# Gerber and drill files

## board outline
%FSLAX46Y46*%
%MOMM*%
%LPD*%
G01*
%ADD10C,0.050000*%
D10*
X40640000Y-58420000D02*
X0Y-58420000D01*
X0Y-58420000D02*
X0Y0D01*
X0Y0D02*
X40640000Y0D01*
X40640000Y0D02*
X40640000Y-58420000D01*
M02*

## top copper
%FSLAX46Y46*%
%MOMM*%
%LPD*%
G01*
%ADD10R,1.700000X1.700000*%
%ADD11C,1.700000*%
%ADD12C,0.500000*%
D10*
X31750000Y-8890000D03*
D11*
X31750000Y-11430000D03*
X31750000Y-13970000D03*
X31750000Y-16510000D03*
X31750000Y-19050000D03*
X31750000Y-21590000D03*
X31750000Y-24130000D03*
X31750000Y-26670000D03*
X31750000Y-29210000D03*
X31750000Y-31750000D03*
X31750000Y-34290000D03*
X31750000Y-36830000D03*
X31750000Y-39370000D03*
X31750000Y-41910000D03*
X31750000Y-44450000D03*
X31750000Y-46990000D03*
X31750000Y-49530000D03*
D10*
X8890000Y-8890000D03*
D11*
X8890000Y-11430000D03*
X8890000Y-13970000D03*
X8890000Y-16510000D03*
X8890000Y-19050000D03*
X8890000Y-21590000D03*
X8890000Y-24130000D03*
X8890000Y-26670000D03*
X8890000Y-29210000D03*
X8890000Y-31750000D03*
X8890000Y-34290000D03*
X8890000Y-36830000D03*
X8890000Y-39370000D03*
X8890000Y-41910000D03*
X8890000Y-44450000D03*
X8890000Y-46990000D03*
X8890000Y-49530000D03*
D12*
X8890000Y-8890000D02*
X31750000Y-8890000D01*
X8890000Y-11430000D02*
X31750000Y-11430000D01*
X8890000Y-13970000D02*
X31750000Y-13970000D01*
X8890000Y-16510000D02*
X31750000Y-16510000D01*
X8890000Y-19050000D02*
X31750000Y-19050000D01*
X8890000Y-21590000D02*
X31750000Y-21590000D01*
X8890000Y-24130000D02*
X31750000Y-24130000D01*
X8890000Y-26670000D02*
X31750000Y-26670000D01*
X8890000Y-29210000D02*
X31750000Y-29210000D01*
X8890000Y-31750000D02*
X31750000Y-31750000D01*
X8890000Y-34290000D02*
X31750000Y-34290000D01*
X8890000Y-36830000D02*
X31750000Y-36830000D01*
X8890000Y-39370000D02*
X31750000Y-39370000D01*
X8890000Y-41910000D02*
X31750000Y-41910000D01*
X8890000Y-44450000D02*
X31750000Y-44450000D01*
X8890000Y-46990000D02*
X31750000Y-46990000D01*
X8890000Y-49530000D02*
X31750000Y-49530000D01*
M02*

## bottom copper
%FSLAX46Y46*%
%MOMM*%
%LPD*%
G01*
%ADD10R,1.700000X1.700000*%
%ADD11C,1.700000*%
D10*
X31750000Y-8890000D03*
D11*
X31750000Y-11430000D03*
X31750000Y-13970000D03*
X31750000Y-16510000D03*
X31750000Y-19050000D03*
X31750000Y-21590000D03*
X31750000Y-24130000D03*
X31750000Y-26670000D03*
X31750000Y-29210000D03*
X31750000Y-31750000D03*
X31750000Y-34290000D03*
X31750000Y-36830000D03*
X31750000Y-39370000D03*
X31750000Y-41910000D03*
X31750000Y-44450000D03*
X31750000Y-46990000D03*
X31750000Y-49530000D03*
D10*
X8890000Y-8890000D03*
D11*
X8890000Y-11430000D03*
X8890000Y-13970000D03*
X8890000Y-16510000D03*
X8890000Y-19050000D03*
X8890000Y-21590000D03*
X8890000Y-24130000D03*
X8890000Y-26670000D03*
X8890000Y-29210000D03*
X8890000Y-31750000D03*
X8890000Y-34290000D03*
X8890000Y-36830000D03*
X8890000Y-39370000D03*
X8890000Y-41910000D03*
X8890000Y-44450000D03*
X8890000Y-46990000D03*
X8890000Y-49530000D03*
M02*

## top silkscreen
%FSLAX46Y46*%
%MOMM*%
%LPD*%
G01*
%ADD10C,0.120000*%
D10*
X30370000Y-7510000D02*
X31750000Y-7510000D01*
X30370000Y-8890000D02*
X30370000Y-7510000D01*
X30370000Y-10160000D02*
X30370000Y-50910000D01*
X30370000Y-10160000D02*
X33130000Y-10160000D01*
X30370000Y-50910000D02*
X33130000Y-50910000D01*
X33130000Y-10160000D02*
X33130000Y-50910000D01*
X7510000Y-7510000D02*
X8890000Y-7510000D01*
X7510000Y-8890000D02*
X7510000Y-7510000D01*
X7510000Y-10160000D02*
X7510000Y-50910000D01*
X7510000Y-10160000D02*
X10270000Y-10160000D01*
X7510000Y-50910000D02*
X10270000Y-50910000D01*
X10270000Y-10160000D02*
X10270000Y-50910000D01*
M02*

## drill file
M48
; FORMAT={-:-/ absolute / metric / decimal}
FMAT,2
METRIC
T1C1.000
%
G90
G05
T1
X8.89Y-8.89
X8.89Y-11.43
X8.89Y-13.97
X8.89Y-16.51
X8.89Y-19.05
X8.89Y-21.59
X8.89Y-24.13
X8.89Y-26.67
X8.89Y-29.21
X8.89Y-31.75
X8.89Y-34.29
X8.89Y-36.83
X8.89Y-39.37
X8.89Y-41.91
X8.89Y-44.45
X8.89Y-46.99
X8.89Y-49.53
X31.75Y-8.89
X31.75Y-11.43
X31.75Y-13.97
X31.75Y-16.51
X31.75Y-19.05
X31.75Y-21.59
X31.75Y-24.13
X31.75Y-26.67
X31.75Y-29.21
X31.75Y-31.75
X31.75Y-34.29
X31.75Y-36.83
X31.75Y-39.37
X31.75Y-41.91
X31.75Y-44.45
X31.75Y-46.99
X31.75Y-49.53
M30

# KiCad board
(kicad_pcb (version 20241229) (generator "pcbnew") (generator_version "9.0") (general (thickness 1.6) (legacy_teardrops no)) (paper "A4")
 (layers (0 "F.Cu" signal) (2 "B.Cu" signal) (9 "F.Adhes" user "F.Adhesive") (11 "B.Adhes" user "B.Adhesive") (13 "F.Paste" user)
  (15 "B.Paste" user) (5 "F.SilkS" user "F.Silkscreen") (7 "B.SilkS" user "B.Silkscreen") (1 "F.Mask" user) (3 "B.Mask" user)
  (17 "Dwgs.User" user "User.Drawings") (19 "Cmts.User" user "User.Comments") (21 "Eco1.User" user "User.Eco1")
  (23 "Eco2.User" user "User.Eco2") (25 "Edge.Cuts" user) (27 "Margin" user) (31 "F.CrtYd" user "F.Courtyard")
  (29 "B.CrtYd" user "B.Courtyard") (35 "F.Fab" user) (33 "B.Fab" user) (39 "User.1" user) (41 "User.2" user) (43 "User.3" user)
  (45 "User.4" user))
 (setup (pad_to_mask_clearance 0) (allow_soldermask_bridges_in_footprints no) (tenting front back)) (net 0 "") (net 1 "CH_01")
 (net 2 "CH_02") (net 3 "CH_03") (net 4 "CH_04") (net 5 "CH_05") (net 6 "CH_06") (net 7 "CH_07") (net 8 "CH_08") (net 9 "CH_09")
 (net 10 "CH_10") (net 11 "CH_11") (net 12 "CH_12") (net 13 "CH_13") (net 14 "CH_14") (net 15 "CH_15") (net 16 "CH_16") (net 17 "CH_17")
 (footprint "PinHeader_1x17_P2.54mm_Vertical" (layer "F.Cu") (at 31.75 8.89)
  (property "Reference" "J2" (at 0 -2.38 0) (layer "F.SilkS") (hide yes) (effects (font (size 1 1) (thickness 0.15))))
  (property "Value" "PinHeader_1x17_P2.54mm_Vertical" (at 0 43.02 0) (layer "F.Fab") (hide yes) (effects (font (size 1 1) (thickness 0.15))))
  (fp_line (start -1.38 -1.38) (end 0 -1.38) (stroke (width 0.12) (type solid)) (layer "F.SilkS"))
  (fp_line (start -1.38 0) (end -1.38 -1.38) (stroke (width 0.12) (type solid)) (layer "F.SilkS"))
  (fp_line (start -1.38 1.27) (end -1.38 42.02) (stroke (width 0.12) (type solid)) (layer "F.SilkS"))
  (fp_line (start -1.38 1.27) (end 1.38 1.27) (stroke (width 0.12) (type solid)) (layer "F.SilkS"))
  (fp_line (start -1.38 42.02) (end 1.38 42.02) (stroke (width 0.12) (type solid)) (layer "F.SilkS"))
  (fp_line (start 1.38 1.27) (end 1.38 42.02) (stroke (width 0.12) (type solid)) (layer "F.SilkS"))
  (pad "1" thru_hole rect (at 0 0) (size 1.7 1.7) (drill 1) (layers "*.Cu" "*.Mask") (remove_unused_layers no) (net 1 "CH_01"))
  (pad "2" thru_hole circle (at 0 2.54) (size 1.7 1.7) (drill 1) (layers "*.Cu" "*.Mask") (remove_unused_layers no) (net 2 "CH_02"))
  (pad "3" thru_hole circle (at 0 5.08) (size 1.7 1.7) (drill 1) (layers "*.Cu" "*.Mask") (remove_unused_layers no) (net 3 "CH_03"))
  (pad "4" thru_hole circle (at 0 7.62) (size 1.7 1.7) (drill 1) (layers "*.Cu" "*.Mask") (remove_unused_layers no) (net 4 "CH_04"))
  (pad "5" thru_hole circle (at 0 10.16) (size 1.7 1.7) (drill 1) (layers "*.Cu" "*.Mask") (remove_unused_layers no) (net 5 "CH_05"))
  (pad "6" thru_hole circle (at 0 12.7) (size 1.7 1.7) (drill 1) (layers "*.Cu" "*.Mask") (remove_unused_layers no) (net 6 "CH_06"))
  (pad "7" thru_hole circle (at 0 15.24) (size 1.7 1.7) (drill 1) (layers "*.Cu" "*.Mask") (remove_unused_layers no) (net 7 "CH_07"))
  (pad "8" thru_hole circle (at 0 17.78) (size 1.7 1.7) (drill 1) (layers "*.Cu" "*.Mask") (remove_unused_layers no) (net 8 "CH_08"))
  (pad "9" thru_hole circle (at 0 20.32) (size 1.7 1.7) (drill 1) (layers "*.Cu" "*.Mask") (remove_unused_layers no) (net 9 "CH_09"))
  (pad "10" thru_hole circle (at 0 22.86) (size 1.7 1.7) (drill 1) (layers "*.Cu" "*.Mask") (remove_unused_layers no) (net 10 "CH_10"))
  (pad "11" thru_hole circle (at 0 25.4) (size 1.7 1.7) (drill 1) (layers "*.Cu" "*.Mask") (remove_unused_layers no) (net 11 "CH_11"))
  (pad "12" thru_hole circle (at 0 27.94) (size 1.7 1.7) (drill 1) (layers "*.Cu" "*.Mask") (remove_unused_layers no) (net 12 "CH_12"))
  (pad "13" thru_hole circle (at 0 30.48) (size 1.7 1.7) (drill 1) (layers "*.Cu" "*.Mask") (remove_unused_layers no) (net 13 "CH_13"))
  (pad "14" thru_hole circle (at 0 33.02) (size 1.7 1.7) (drill 1) (layers "*.Cu" "*.Mask") (remove_unused_layers no) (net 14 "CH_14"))
  (pad "15" thru_hole circle (at 0 35.56) (size 1.7 1.7) (drill 1) (layers "*.Cu" "*.Mask") (remove_unused_layers no) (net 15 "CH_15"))
  (pad "16" thru_hole circle (at 0 38.1) (size 1.7 1.7) (drill 1) (layers "*.Cu" "*.Mask") (remove_unused_layers no) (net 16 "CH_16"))
  (pad "17" thru_hole circle (at 0 40.64) (size 1.7 1.7) (drill 1) (layers "*.Cu" "*.Mask") (remove_unused_layers no) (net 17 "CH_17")))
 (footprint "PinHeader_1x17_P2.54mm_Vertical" (layer "F.Cu") (at 8.89 8.89)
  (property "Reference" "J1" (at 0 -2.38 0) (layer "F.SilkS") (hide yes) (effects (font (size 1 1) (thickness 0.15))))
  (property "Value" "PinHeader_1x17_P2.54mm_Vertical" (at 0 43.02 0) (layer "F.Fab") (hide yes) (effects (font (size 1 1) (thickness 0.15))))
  (fp_line (start -1.38 -1.38) (end 0 -1.38) (stroke (width 0.12) (type solid)) (layer "F.SilkS"))
  (fp_line (start -1.38 0) (end -1.38 -1.38) (stroke (width 0.12) (type solid)) (layer "F.SilkS"))
  (fp_line (start -1.38 1.27) (end -1.38 42.02) (stroke (width 0.12) (type solid)) (layer "F.SilkS"))
  (fp_line (start -1.38 1.27) (end 1.38 1.27) (stroke (width 0.12) (type solid)) (layer "F.SilkS"))
  (fp_line (start -1.38 42.02) (end 1.38 42.02) (stroke (width 0.12) (type solid)) (layer "F.SilkS"))
  (fp_line (start 1.38 1.27) (end 1.38 42.02) (stroke (width 0.12) (type solid)) (layer "F.SilkS"))
  (pad "1" thru_hole rect (at 0 0) (size 1.7 1.7) (drill 1) (layers "*.Cu" "*.Mask") (remove_unused_layers no) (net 1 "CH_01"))
  (pad "2" thru_hole circle (at 0 2.54) (size 1.7 1.7) (drill 1) (layers "*.Cu" "*.Mask") (remove_unused_layers no) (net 2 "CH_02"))
  (pad "3" thru_hole circle (at 0 5.08) (size 1.7 1.7) (drill 1) (layers "*.Cu" "*.Mask") (remove_unused_layers no) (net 3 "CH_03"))
  (pad "4" thru_hole circle (at 0 7.62) (size 1.7 1.7) (drill 1) (layers "*.Cu" "*.Mask") (remove_unused_layers no) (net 4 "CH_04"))
  (pad "5" thru_hole circle (at 0 10.16) (size 1.7 1.7) (drill 1) (layers "*.Cu" "*.Mask") (remove_unused_layers no) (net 5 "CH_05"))
  (pad "6" thru_hole circle (at 0 12.7) (size 1.7 1.7) (drill 1) (layers "*.Cu" "*.Mask") (remove_unused_layers no) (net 6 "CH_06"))
  (pad "7" thru_hole circle (at 0 15.24) (size 1.7 1.7) (drill 1) (layers "*.Cu" "*.Mask") (remove_unused_layers no) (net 7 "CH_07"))
  (pad "8" thru_hole circle (at 0 17.78) (size 1.7 1.7) (drill 1) (layers "*.Cu" "*.Mask") (remove_unused_layers no) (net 8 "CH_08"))
  (pad "9" thru_hole circle (at 0 20.32) (size 1.7 1.7) (drill 1) (layers "*.Cu" "*.Mask") (remove_unused_layers no) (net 9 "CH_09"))
  (pad "10" thru_hole circle (at 0 22.86) (size 1.7 1.7) (drill 1) (layers "*.Cu" "*.Mask") (remove_unused_layers no) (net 10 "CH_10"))
  (pad "11" thru_hole circle (at 0 25.4) (size 1.7 1.7) (drill 1) (layers "*.Cu" "*.Mask") (remove_unused_layers no) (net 11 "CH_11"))
  (pad "12" thru_hole circle (at 0 27.94) (size 1.7 1.7) (drill 1) (layers "*.Cu" "*.Mask") (remove_unused_layers no) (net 12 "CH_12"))
  (pad "13" thru_hole circle (at 0 30.48) (size 1.7 1.7) (drill 1) (layers "*.Cu" "*.Mask") (remove_unused_layers no) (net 13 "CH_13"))
  (pad "14" thru_hole circle (at 0 33.02) (size 1.7 1.7) (drill 1) (layers "*.Cu" "*.Mask") (remove_unused_layers no) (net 14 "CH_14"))
  (pad "15" thru_hole circle (at 0 35.56) (size 1.7 1.7) (drill 1) (layers "*.Cu" "*.Mask") (remove_unused_layers no) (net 15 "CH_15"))
  (pad "16" thru_hole circle (at 0 38.1) (size 1.7 1.7) (drill 1) (layers "*.Cu" "*.Mask") (remove_unused_layers no) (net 16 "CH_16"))
  (pad "17" thru_hole circle (at 0 40.64) (size 1.7 1.7) (drill 1) (layers "*.Cu" "*.Mask") (remove_unused_layers no) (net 17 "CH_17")))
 (gr_line (start 40.64 58.42) (end 0 58.42) (stroke (width 0.05) (type default)) (layer "Edge.Cuts"))
 (gr_line (start 0 58.42) (end 0 0) (stroke (width 0.05) (type default)) (layer "Edge.Cuts"))
 (gr_line (start 0 0) (end 40.64 0) (stroke (width 0.05) (type default)) (layer "Edge.Cuts"))
 (gr_line (start 40.64 0) (end 40.64 58.42) (stroke (width 0.05) (type default)) (layer "Edge.Cuts"))
 (segment (start 8.89 8.89) (end 31.75 8.89) (width 0.5) (layer "F.Cu") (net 1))
 (segment (start 8.89 11.43) (end 31.75 11.43) (width 0.5) (layer "F.Cu") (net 2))
 (segment (start 8.89 13.97) (end 31.75 13.97) (width 0.5) (layer "F.Cu") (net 3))
 (segment (start 8.89 16.51) (end 31.75 16.51) (width 0.5) (layer "F.Cu") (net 4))
 (segment (start 8.89 19.05) (end 31.75 19.05) (width 0.5) (layer "F.Cu") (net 5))
 (segment (start 8.89 21.59) (end 31.75 21.59) (width 0.5) (layer "F.Cu") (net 6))
 (segment (start 8.89 24.13) (end 31.75 24.13) (width 0.5) (layer "F.Cu") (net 7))
 (segment (start 8.89 26.67) (end 31.75 26.67) (width 0.5) (layer "F.Cu") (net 8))
 (segment (start 8.89 29.21) (end 31.75 29.21) (width 0.5) (layer "F.Cu") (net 9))
 (segment (start 8.89 31.75) (end 31.75 31.75) (width 0.5) (layer "F.Cu") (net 10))
 (segment (start 8.89 34.29) (end 31.75 34.29) (width 0.5) (layer "F.Cu") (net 11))
 (segment (start 8.89 36.83) (end 31.75 36.83) (width 0.5) (layer "F.Cu") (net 12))
 (segment (start 8.89 39.37) (end 31.75 39.37) (width 0.5) (layer "F.Cu") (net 13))
 (segment (start 8.89 41.91) (end 31.75 41.91) (width 0.5) (layer "F.Cu") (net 14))
 (segment (start 8.89 44.45) (end 31.75 44.45) (width 0.5) (layer "F.Cu") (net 15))
 (segment (start 8.89 46.99) (end 31.75 46.99) (width 0.5) (layer "F.Cu") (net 16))
 (segment (start 8.89 49.53) (end 31.75 49.53) (width 0.5) (layer "F.Cu") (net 17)))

